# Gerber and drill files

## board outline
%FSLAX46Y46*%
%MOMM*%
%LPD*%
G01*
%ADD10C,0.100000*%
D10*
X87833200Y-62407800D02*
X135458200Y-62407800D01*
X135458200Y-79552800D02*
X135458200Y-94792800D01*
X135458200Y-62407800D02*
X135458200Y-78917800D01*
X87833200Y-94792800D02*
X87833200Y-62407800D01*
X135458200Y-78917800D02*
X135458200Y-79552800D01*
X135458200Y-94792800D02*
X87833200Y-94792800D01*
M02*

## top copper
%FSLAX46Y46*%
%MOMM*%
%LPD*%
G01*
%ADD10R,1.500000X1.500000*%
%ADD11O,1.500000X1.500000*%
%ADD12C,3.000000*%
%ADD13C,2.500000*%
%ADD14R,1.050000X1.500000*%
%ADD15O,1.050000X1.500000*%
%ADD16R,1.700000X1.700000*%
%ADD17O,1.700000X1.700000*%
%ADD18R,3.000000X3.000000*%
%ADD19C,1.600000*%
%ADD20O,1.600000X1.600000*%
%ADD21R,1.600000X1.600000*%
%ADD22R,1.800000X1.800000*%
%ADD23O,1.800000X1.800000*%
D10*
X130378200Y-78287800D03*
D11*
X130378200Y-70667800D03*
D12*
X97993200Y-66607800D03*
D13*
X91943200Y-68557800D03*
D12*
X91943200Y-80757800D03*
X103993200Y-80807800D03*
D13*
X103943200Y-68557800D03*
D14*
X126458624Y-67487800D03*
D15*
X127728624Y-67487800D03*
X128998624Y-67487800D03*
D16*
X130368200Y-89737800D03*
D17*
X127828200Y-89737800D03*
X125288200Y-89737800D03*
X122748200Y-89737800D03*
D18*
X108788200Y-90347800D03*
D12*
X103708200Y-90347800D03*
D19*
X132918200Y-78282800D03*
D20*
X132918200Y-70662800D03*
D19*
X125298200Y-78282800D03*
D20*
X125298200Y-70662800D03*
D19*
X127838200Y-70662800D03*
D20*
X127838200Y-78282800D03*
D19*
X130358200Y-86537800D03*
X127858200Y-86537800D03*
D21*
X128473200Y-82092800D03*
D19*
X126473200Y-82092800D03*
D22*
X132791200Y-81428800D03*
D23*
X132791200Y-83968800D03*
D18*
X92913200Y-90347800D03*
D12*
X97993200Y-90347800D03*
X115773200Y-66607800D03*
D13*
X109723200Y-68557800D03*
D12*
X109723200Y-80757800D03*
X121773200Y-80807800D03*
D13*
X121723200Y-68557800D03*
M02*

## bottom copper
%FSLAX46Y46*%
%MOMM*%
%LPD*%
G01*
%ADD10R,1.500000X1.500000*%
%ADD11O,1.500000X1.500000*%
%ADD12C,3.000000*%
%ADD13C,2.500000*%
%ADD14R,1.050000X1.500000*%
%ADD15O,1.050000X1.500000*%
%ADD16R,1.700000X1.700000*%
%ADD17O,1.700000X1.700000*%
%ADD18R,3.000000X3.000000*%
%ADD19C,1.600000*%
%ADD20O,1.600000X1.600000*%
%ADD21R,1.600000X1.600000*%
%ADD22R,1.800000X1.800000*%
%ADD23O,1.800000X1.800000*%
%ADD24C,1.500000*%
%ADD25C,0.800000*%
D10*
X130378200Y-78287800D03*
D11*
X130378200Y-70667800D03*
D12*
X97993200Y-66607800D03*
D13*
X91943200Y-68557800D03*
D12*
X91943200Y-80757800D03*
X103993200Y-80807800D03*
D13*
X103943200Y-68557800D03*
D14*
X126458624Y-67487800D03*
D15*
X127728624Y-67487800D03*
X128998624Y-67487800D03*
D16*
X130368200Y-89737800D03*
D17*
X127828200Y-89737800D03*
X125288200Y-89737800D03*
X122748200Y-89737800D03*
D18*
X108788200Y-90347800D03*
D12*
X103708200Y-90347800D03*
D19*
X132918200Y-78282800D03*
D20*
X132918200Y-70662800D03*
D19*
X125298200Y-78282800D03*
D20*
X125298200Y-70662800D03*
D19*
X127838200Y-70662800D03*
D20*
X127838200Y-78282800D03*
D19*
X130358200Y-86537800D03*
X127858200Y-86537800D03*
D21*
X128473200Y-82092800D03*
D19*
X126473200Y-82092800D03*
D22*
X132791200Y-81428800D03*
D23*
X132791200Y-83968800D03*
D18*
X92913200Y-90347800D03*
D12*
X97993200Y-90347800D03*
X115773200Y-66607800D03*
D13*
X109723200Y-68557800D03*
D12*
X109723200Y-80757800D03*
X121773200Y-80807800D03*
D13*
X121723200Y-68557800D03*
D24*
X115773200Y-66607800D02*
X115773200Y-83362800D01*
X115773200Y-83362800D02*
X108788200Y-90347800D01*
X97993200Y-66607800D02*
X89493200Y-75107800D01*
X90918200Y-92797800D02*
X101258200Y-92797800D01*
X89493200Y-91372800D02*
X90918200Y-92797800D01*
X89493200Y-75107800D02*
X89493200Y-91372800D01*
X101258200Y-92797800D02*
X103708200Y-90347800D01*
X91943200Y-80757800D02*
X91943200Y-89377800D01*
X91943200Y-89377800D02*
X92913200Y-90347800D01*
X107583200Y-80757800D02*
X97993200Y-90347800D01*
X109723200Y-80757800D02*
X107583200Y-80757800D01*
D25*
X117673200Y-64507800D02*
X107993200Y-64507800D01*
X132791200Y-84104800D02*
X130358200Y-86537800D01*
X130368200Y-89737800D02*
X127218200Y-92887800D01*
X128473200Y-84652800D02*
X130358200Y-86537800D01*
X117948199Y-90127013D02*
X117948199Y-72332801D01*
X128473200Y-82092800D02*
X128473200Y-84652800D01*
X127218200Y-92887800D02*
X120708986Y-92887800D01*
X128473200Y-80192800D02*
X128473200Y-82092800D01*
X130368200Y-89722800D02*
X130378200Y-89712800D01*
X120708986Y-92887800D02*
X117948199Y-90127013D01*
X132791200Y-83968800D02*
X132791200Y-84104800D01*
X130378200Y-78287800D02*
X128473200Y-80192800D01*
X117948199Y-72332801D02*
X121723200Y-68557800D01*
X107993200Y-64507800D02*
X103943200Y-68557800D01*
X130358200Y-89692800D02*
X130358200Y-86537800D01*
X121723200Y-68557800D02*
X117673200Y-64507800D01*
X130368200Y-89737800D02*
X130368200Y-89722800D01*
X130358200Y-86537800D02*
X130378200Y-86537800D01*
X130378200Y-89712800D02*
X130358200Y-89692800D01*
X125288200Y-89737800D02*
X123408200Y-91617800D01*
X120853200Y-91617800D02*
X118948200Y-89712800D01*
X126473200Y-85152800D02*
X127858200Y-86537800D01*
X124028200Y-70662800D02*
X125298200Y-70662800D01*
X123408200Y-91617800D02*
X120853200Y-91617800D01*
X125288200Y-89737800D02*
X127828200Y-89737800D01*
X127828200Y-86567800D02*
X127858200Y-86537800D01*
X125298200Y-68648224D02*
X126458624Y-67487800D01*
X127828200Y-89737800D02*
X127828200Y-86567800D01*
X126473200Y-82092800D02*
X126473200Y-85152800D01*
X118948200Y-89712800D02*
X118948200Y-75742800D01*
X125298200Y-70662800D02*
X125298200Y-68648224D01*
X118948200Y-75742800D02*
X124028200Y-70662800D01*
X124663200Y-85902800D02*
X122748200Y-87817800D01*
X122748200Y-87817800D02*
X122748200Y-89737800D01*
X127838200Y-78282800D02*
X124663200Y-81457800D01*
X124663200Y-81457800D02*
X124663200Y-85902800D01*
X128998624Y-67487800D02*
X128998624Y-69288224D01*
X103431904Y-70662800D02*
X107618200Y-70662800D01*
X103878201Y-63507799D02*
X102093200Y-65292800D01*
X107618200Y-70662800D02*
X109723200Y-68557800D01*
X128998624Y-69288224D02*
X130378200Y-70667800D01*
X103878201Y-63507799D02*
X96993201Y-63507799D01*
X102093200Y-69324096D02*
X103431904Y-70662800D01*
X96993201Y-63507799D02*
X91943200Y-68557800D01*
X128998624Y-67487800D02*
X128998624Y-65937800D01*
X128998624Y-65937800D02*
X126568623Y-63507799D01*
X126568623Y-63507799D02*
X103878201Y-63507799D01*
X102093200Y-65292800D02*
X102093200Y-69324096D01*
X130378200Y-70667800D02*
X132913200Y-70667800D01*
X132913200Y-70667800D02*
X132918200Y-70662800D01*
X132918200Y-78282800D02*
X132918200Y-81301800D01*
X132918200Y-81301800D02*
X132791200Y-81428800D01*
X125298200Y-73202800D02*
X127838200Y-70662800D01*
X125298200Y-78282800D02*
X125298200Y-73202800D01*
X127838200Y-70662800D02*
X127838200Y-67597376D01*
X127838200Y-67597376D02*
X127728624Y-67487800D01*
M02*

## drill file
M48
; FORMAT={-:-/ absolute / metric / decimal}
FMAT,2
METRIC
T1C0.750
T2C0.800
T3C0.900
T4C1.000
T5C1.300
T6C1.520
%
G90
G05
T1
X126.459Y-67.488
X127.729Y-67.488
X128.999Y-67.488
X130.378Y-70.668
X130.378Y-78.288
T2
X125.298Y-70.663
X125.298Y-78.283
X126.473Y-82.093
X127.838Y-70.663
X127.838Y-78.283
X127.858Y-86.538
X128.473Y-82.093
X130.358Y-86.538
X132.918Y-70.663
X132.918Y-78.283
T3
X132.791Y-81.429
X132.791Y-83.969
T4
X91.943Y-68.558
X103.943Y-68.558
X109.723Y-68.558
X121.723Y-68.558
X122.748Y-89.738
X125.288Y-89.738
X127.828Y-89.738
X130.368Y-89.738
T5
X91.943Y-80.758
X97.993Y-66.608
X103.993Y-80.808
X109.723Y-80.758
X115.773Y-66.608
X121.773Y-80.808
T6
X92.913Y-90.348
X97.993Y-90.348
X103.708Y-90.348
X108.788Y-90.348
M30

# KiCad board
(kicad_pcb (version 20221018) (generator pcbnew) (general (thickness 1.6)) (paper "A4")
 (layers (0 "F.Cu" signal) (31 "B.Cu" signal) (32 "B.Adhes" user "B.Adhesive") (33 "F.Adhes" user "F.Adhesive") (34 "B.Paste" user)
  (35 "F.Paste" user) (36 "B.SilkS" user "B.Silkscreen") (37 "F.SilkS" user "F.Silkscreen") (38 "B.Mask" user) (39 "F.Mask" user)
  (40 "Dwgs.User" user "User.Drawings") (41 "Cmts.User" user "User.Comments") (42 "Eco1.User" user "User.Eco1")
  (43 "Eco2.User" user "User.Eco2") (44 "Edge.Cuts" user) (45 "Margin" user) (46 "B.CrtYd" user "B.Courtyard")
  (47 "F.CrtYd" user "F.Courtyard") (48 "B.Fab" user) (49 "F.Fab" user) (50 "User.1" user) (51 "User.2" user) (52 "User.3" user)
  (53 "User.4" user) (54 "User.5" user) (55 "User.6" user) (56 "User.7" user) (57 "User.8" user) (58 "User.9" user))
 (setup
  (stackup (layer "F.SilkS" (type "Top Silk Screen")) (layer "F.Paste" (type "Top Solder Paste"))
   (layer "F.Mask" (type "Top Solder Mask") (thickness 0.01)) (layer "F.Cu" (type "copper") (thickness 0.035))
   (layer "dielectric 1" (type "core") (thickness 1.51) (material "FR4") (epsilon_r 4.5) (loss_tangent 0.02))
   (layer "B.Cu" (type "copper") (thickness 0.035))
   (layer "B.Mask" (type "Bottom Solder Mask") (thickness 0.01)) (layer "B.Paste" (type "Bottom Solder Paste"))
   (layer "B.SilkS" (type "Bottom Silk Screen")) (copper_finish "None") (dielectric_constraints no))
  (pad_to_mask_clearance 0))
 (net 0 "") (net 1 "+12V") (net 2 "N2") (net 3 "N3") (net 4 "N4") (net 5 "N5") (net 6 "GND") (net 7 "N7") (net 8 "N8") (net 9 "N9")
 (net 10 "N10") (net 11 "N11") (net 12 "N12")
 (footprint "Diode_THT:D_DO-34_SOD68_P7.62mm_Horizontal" (layer "F.Cu") (at 130.3782 78.2878 90)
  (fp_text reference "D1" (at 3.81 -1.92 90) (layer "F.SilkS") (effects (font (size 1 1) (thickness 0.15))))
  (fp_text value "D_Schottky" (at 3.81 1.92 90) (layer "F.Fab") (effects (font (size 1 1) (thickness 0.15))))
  (pad "1" thru_hole rect (at 0 0 90) (size 1.5 1.5) (drill 0.75) (layers "*.Cu" "*.Mask") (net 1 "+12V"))
  (pad "2" thru_hole oval (at 7.62 0 90) (size 1.5 1.5) (drill 0.75) (layers "*.Cu" "*.Mask") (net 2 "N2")))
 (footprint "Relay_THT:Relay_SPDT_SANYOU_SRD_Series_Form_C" (layer "F.Cu") (at 97.9932 66.6078 -90)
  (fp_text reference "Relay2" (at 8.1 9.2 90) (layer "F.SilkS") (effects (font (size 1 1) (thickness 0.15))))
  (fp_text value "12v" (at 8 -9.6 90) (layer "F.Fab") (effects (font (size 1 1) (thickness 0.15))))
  (pad "1" thru_hole circle (at 0 0) (size 3 3) (drill 1.3) (layers "*.Cu" "*.Mask") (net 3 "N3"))
  (pad "2" thru_hole circle (at 1.95 6.05) (size 2.5 2.5) (drill 1) (layers "*.Cu" "*.Mask") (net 2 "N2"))
  (pad "3" thru_hole circle (at 14.15 6.05) (size 3 3) (drill 1.3) (layers "*.Cu" "*.Mask") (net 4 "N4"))
  (pad "4" thru_hole circle (at 14.2 -6) (size 3 3) (drill 1.3) (layers "*.Cu" "*.Mask") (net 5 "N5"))
  (pad "5" thru_hole circle (at 1.95 -5.95) (size 2.5 2.5) (drill 1) (layers "*.Cu" "*.Mask") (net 1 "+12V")))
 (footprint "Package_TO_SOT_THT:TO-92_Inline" (layer "F.Cu") (at 126.458624 67.4878)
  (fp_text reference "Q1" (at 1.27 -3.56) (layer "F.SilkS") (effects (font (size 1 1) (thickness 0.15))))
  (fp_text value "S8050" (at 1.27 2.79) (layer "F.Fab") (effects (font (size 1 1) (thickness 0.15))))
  (pad "1" thru_hole rect (at 0 0) (size 1.05 1.5) (drill 0.75) (layers "*.Cu" "*.Mask") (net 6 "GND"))
  (pad "2" thru_hole oval (at 1.27 0) (size 1.05 1.5) (drill 0.75) (layers "*.Cu" "*.Mask") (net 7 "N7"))
  (pad "3" thru_hole oval (at 2.54 0) (size 1.05 1.5) (drill 0.75) (layers "*.Cu" "*.Mask") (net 2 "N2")))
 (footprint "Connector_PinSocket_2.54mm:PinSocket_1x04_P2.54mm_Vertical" (layer "F.Cu") (at 130.3682 89.7378 -90)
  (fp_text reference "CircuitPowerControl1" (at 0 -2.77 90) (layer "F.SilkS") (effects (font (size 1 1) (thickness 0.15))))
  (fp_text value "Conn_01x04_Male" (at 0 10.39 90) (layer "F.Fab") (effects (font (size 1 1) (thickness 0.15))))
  (pad "1" thru_hole rect (at 0 0 270) (size 1.7 1.7) (drill 1) (layers "*.Cu" "*.Mask") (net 1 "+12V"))
  (pad "2" thru_hole oval (at 0 2.54 270) (size 1.7 1.7) (drill 1) (layers "*.Cu" "*.Mask") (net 6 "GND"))
  (pad "3" thru_hole oval (at 0 5.08 270) (size 1.7 1.7) (drill 1) (layers "*.Cu" "*.Mask") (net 6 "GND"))
  (pad "4" thru_hole oval (at 0 7.62 270) (size 1.7 1.7) (drill 1) (layers "*.Cu" "*.Mask") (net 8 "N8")))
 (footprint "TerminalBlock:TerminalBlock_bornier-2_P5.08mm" (layer "F.Cu") (at 108.7882 90.3478 180)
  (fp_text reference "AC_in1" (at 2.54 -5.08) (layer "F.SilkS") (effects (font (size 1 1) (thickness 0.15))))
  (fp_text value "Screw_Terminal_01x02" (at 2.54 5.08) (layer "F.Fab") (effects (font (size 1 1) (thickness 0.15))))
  (pad "1" thru_hole rect (at 0 0 180) (size 3 3) (drill 1.52) (layers "*.Cu" "*.Mask") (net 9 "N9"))
  (pad "2" thru_hole circle (at 5.08 0 180) (size 3 3) (drill 1.52) (layers "*.Cu" "*.Mask") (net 3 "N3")))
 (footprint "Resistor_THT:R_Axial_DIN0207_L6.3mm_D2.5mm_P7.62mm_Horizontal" (layer "F.Cu") (at 132.9182 78.2828 90)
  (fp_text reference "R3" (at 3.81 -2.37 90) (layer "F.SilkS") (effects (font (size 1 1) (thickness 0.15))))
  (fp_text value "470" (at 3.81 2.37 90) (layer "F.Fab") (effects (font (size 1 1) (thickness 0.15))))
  (pad "1" thru_hole circle (at 0 0 90) (size 1.6 1.6) (drill 0.8) (layers "*.Cu" "*.Mask") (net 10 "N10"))
  (pad "2" thru_hole oval (at 7.62 0 90) (size 1.6 1.6) (drill 0.8) (layers "*.Cu" "*.Mask") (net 2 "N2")))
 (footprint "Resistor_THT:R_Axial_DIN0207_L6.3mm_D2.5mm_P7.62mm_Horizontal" (layer "F.Cu") (at 125.2982 78.2828 90)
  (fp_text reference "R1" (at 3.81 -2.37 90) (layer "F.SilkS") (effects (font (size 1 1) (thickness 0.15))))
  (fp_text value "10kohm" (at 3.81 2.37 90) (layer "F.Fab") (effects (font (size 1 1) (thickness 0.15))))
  (pad "1" thru_hole circle (at 0 0 90) (size 1.6 1.6) (drill 0.8) (layers "*.Cu" "*.Mask") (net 7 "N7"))
  (pad "2" thru_hole oval (at 7.62 0 90) (size 1.6 1.6) (drill 0.8) (layers "*.Cu" "*.Mask") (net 6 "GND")))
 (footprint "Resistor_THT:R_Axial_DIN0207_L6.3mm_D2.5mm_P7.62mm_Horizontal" (layer "F.Cu") (at 127.8382 70.6628 -90)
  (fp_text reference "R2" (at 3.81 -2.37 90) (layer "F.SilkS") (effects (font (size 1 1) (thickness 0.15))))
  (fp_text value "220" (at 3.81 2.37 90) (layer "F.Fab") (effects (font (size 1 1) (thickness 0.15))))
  (pad "1" thru_hole circle (at 0 0 270) (size 1.6 1.6) (drill 0.8) (layers "*.Cu" "*.Mask") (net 7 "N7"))
  (pad "2" thru_hole oval (at 7.62 0 270) (size 1.6 1.6) (drill 0.8) (layers "*.Cu" "*.Mask") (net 8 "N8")))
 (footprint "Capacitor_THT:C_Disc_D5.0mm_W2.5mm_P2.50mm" (layer "F.Cu") (at 130.3582 86.5378 180)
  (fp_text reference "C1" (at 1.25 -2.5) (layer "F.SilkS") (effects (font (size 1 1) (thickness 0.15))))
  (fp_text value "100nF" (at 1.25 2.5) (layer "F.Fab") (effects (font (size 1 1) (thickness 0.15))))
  (pad "1" thru_hole circle (at 0 0 180) (size 1.6 1.6) (drill 0.8) (layers "*.Cu" "*.Mask") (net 1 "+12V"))
  (pad "2" thru_hole circle (at 2.5 0 180) (size 1.6 1.6) (drill 0.8) (layers "*.Cu" "*.Mask") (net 6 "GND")))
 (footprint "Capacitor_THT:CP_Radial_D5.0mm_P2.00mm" (layer "F.Cu") (at 128.4732 82.0928 180)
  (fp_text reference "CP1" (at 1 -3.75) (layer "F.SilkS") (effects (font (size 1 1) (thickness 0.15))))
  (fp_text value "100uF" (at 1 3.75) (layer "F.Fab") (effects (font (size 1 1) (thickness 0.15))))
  (pad "1" thru_hole rect (at 0 0 180) (size 1.6 1.6) (drill 0.8) (layers "*.Cu" "*.Mask") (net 1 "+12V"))
  (pad "2" thru_hole circle (at 2 0 180) (size 1.6 1.6) (drill 0.8) (layers "*.Cu" "*.Mask") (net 6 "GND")))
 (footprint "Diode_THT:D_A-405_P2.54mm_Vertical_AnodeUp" (layer "F.Cu") (at 132.7912 81.4288 -90)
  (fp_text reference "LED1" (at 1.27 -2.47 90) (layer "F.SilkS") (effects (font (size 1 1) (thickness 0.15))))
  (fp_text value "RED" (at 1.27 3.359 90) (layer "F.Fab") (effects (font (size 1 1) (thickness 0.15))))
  (pad "1" thru_hole rect (at 0 0 270) (size 1.8 1.8) (drill 0.9) (layers "*.Cu" "*.Mask") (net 10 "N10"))
  (pad "2" thru_hole oval (at 2.54 0 270) (size 1.8 1.8) (drill 0.9) (layers "*.Cu" "*.Mask") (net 1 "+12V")))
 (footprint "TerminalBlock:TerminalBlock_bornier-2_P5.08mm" (layer "F.Cu") (at 92.9132 90.3478)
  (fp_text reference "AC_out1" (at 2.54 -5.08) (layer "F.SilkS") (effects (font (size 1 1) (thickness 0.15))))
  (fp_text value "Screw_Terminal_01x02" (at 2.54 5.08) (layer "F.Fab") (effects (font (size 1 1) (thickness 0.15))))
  (pad "1" thru_hole rect (at 0 0) (size 3 3) (drill 1.52) (layers "*.Cu" "*.Mask") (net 4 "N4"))
  (pad "2" thru_hole circle (at 5.08 0) (size 3 3) (drill 1.52) (layers "*.Cu" "*.Mask") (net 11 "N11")))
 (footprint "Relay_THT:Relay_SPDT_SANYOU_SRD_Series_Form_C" (layer "F.Cu") (at 115.7732 66.6078 -90)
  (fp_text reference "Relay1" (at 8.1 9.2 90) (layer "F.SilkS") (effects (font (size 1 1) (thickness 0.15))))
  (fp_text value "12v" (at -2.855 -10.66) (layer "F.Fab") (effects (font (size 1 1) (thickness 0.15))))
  (pad "1" thru_hole circle (at 0 0) (size 3 3) (drill 1.3) (layers "*.Cu" "*.Mask") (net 9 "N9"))
  (pad "2" thru_hole circle (at 1.95 6.05) (size 2.5 2.5) (drill 1) (layers "*.Cu" "*.Mask") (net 2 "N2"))
  (pad "3" thru_hole circle (at 14.15 6.05) (size 3 3) (drill 1.3) (layers "*.Cu" "*.Mask") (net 11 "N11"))
  (pad "4" thru_hole circle (at 14.2 -6) (size 3 3) (drill 1.3) (layers "*.Cu" "*.Mask") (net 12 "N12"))
  (pad "5" thru_hole circle (at 1.95 -5.95) (size 2.5 2.5) (drill 1) (layers "*.Cu" "*.Mask") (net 1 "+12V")))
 (gr_line (start 87.8332 62.4078) (end 135.4582 62.4078) (stroke (width 0.1) (type solid)) (layer "Edge.Cuts"))
 (gr_line (start 135.4582 79.5528) (end 135.4582 94.7928) (stroke (width 0.1) (type solid)) (layer "Edge.Cuts"))
 (gr_line (start 135.4582 62.4078) (end 135.4582 78.9178) (stroke (width 0.1) (type solid)) (layer "Edge.Cuts"))
 (gr_line (start 87.8332 94.7928) (end 87.8332 62.4078) (stroke (width 0.1) (type solid)) (layer "Edge.Cuts"))
 (gr_line (start 135.4582 78.9178) (end 135.4582 79.5528) (stroke (width 0.1) (type solid)) (layer "Edge.Cuts"))
 (gr_line (start 135.4582 94.7928) (end 87.8332 94.7928) (stroke (width 0.1) (type solid)) (layer "Edge.Cuts"))
 (segment (start 115.7732 66.6078) (end 115.7732 83.3628) (width 1.5) (layer "B.Cu") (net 9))
 (segment (start 115.7732 83.3628) (end 108.7882 90.3478) (width 1.5) (layer "B.Cu") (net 9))
 (segment (start 97.9932 66.6078) (end 89.4932 75.1078) (width 1.5) (layer "B.Cu") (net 3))
 (segment (start 90.9182 92.7978) (end 101.2582 92.7978) (width 1.5) (layer "B.Cu") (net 3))
 (segment (start 89.4932 91.3728) (end 90.9182 92.7978) (width 1.5) (layer "B.Cu") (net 3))
 (segment (start 89.4932 75.1078) (end 89.4932 91.3728) (width 1.5) (layer "B.Cu") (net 3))
 (segment (start 101.2582 92.7978) (end 103.7082 90.3478) (width 1.5) (layer "B.Cu") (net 3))
 (segment (start 91.9432 80.7578) (end 91.9432 89.3778) (width 1.5) (layer "B.Cu") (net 4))
 (segment (start 91.9432 89.3778) (end 92.9132 90.3478) (width 1.5) (layer "B.Cu") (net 4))
 (segment (start 107.5832 80.7578) (end 97.9932 90.3478) (width 1.5) (layer "B.Cu") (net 11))
 (segment (start 109.7232 80.7578) (end 107.5832 80.7578) (width 1.5) (layer "B.Cu") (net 11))
 (segment (start 117.6732 64.5078) (end 107.9932 64.5078) (width 0.8) (layer "B.Cu") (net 1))
 (segment (start 132.7912 84.1048) (end 130.3582 86.5378) (width 0.8) (layer "B.Cu") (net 1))
 (segment (start 130.3682 89.7378) (end 127.2182 92.8878) (width 0.8) (layer "B.Cu") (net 1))
 (segment (start 128.4732 84.6528) (end 130.3582 86.5378) (width 0.8) (layer "B.Cu") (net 1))
 (segment (start 117.948199 90.127013) (end 117.948199 72.332801) (width 0.8) (layer "B.Cu") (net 1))
 (segment (start 128.4732 82.0928) (end 128.4732 84.6528) (width 0.8) (layer "B.Cu") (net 1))
 (segment (start 127.2182 92.8878) (end 120.708986 92.8878) (width 0.8) (layer "B.Cu") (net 1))
 (segment (start 128.4732 80.1928) (end 128.4732 82.0928) (width 0.8) (layer "B.Cu") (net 1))
 (segment (start 130.3682 89.7228) (end 130.3782 89.7128) (width 0.8) (layer "B.Cu") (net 1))
 (segment (start 120.708986 92.8878) (end 117.948199 90.127013) (width 0.8) (layer "B.Cu") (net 1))
 (segment (start 132.7912 83.9688) (end 132.7912 84.1048) (width 0.8) (layer "B.Cu") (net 1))
 (segment (start 130.3782 78.2878) (end 128.4732 80.1928) (width 0.8) (layer "B.Cu") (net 1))
 (segment (start 117.948199 72.332801) (end 121.7232 68.5578) (width 0.8) (layer "B.Cu") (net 1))
 (segment (start 107.9932 64.5078) (end 103.9432 68.5578) (width 0.8) (layer "B.Cu") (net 1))
 (segment (start 130.3582 89.6928) (end 130.3582 86.5378) (width 0.8) (layer "B.Cu") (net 1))
 (segment (start 121.7232 68.5578) (end 117.6732 64.5078) (width 0.8) (layer "B.Cu") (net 1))
 (segment (start 130.3682 89.7378) (end 130.3682 89.7228) (width 0.8) (layer "B.Cu") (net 1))
 (segment (start 130.3582 86.5378) (end 130.3782 86.5378) (width 0.8) (layer "B.Cu") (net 1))
 (segment (start 130.3782 89.7128) (end 130.3582 89.6928) (width 0.8) (layer "B.Cu") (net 1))
 (segment (start 125.2882 89.7378) (end 123.4082 91.6178) (width 0.8) (layer "B.Cu") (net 6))
 (segment (start 120.8532 91.6178) (end 118.9482 89.7128) (width 0.8) (layer "B.Cu") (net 6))
 (segment (start 126.4732 85.1528) (end 127.8582 86.5378) (width 0.8) (layer "B.Cu") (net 6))
 (segment (start 124.0282 70.6628) (end 125.2982 70.6628) (width 0.8) (layer "B.Cu") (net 6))
 (segment (start 123.4082 91.6178) (end 120.8532 91.6178) (width 0.8) (layer "B.Cu") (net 6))
 (segment (start 125.2882 89.7378) (end 127.8282 89.7378) (width 0.8) (layer "B.Cu") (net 6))
 (segment (start 127.8282 86.5678) (end 127.8582 86.5378) (width 0.8) (layer "B.Cu") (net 6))
 (segment (start 125.2982 68.648224) (end 126.458624 67.4878) (width 0.8) (layer "B.Cu") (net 6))
 (segment (start 127.8282 89.7378) (end 127.8282 86.5678) (width 0.8) (layer "B.Cu") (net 6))
 (segment (start 126.4732 82.0928) (end 126.4732 85.1528) (width 0.8) (layer "B.Cu") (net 6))
 (segment (start 118.9482 89.7128) (end 118.9482 75.7428) (width 0.8) (layer "B.Cu") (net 6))
 (segment (start 125.2982 70.6628) (end 125.2982 68.648224) (width 0.8) (layer "B.Cu") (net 6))
 (segment (start 118.9482 75.7428) (end 124.0282 70.6628) (width 0.8) (layer "B.Cu") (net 6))
 (segment (start 124.6632 85.9028) (end 122.7482 87.8178) (width 0.8) (layer "B.Cu") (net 8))
 (segment (start 122.7482 87.8178) (end 122.7482 89.7378) (width 0.8) (layer "B.Cu") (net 8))
 (segment (start 127.8382 78.2828) (end 124.6632 81.4578) (width 0.8) (layer "B.Cu") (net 8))
 (segment (start 124.6632 81.4578) (end 124.6632 85.9028) (width 0.8) (layer "B.Cu") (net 8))
 (segment (start 128.998624 67.4878) (end 128.998624 69.288224) (width 0.8) (layer "B.Cu") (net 2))
 (segment (start 103.431904 70.6628) (end 107.6182 70.6628) (width 0.8) (layer "B.Cu") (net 2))
 (segment (start 103.878201 63.507799) (end 102.0932 65.2928) (width 0.8) (layer "B.Cu") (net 2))
 (segment (start 107.6182 70.6628) (end 109.7232 68.5578) (width 0.8) (layer "B.Cu") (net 2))
 (segment (start 128.998624 69.288224) (end 130.3782 70.6678) (width 0.8) (layer "B.Cu") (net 2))
 (segment (start 103.878201 63.507799) (end 96.993201 63.507799) (width 0.8) (layer "B.Cu") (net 2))
 (segment (start 102.0932 69.324096) (end 103.431904 70.6628) (width 0.8) (layer "B.Cu") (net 2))
 (segment (start 96.993201 63.507799) (end 91.9432 68.5578) (width 0.8) (layer "B.Cu") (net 2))
 (segment (start 128.998624 67.4878) (end 128.998624 65.9378) (width 0.8) (layer "B.Cu") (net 2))
 (segment (start 128.998624 65.9378) (end 126.568623 63.507799) (width 0.8) (layer "B.Cu") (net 2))
 (segment (start 126.568623 63.507799) (end 103.878201 63.507799) (width 0.8) (layer "B.Cu") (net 2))
 (segment (start 102.0932 65.2928) (end 102.0932 69.324096) (width 0.8) (layer "B.Cu") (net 2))
 (segment (start 130.3782 70.6678) (end 132.9132 70.6678) (width 0.8) (layer "B.Cu") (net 2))
 (segment (start 132.9132 70.6678) (end 132.9182 70.6628) (width 0.8) (layer "B.Cu") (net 2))
 (segment (start 132.9182 78.2828) (end 132.9182 81.3018) (width 0.8) (layer "B.Cu") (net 10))
 (segment (start 132.9182 81.3018) (end 132.7912 81.4288) (width 0.8) (layer "B.Cu") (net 10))
 (segment (start 125.2982 73.2028) (end 127.8382 70.6628) (width 0.8) (layer "B.Cu") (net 7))
 (segment (start 125.2982 78.2828) (end 125.2982 73.2028) (width 0.8) (layer "B.Cu") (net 7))
 (segment (start 127.8382 70.6628) (end 127.8382 67.597376) (width 0.8) (layer "B.Cu") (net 7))
 (segment (start 127.8382 67.597376) (end 127.728624 67.4878) (width 0.8) (layer "B.Cu") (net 7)))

